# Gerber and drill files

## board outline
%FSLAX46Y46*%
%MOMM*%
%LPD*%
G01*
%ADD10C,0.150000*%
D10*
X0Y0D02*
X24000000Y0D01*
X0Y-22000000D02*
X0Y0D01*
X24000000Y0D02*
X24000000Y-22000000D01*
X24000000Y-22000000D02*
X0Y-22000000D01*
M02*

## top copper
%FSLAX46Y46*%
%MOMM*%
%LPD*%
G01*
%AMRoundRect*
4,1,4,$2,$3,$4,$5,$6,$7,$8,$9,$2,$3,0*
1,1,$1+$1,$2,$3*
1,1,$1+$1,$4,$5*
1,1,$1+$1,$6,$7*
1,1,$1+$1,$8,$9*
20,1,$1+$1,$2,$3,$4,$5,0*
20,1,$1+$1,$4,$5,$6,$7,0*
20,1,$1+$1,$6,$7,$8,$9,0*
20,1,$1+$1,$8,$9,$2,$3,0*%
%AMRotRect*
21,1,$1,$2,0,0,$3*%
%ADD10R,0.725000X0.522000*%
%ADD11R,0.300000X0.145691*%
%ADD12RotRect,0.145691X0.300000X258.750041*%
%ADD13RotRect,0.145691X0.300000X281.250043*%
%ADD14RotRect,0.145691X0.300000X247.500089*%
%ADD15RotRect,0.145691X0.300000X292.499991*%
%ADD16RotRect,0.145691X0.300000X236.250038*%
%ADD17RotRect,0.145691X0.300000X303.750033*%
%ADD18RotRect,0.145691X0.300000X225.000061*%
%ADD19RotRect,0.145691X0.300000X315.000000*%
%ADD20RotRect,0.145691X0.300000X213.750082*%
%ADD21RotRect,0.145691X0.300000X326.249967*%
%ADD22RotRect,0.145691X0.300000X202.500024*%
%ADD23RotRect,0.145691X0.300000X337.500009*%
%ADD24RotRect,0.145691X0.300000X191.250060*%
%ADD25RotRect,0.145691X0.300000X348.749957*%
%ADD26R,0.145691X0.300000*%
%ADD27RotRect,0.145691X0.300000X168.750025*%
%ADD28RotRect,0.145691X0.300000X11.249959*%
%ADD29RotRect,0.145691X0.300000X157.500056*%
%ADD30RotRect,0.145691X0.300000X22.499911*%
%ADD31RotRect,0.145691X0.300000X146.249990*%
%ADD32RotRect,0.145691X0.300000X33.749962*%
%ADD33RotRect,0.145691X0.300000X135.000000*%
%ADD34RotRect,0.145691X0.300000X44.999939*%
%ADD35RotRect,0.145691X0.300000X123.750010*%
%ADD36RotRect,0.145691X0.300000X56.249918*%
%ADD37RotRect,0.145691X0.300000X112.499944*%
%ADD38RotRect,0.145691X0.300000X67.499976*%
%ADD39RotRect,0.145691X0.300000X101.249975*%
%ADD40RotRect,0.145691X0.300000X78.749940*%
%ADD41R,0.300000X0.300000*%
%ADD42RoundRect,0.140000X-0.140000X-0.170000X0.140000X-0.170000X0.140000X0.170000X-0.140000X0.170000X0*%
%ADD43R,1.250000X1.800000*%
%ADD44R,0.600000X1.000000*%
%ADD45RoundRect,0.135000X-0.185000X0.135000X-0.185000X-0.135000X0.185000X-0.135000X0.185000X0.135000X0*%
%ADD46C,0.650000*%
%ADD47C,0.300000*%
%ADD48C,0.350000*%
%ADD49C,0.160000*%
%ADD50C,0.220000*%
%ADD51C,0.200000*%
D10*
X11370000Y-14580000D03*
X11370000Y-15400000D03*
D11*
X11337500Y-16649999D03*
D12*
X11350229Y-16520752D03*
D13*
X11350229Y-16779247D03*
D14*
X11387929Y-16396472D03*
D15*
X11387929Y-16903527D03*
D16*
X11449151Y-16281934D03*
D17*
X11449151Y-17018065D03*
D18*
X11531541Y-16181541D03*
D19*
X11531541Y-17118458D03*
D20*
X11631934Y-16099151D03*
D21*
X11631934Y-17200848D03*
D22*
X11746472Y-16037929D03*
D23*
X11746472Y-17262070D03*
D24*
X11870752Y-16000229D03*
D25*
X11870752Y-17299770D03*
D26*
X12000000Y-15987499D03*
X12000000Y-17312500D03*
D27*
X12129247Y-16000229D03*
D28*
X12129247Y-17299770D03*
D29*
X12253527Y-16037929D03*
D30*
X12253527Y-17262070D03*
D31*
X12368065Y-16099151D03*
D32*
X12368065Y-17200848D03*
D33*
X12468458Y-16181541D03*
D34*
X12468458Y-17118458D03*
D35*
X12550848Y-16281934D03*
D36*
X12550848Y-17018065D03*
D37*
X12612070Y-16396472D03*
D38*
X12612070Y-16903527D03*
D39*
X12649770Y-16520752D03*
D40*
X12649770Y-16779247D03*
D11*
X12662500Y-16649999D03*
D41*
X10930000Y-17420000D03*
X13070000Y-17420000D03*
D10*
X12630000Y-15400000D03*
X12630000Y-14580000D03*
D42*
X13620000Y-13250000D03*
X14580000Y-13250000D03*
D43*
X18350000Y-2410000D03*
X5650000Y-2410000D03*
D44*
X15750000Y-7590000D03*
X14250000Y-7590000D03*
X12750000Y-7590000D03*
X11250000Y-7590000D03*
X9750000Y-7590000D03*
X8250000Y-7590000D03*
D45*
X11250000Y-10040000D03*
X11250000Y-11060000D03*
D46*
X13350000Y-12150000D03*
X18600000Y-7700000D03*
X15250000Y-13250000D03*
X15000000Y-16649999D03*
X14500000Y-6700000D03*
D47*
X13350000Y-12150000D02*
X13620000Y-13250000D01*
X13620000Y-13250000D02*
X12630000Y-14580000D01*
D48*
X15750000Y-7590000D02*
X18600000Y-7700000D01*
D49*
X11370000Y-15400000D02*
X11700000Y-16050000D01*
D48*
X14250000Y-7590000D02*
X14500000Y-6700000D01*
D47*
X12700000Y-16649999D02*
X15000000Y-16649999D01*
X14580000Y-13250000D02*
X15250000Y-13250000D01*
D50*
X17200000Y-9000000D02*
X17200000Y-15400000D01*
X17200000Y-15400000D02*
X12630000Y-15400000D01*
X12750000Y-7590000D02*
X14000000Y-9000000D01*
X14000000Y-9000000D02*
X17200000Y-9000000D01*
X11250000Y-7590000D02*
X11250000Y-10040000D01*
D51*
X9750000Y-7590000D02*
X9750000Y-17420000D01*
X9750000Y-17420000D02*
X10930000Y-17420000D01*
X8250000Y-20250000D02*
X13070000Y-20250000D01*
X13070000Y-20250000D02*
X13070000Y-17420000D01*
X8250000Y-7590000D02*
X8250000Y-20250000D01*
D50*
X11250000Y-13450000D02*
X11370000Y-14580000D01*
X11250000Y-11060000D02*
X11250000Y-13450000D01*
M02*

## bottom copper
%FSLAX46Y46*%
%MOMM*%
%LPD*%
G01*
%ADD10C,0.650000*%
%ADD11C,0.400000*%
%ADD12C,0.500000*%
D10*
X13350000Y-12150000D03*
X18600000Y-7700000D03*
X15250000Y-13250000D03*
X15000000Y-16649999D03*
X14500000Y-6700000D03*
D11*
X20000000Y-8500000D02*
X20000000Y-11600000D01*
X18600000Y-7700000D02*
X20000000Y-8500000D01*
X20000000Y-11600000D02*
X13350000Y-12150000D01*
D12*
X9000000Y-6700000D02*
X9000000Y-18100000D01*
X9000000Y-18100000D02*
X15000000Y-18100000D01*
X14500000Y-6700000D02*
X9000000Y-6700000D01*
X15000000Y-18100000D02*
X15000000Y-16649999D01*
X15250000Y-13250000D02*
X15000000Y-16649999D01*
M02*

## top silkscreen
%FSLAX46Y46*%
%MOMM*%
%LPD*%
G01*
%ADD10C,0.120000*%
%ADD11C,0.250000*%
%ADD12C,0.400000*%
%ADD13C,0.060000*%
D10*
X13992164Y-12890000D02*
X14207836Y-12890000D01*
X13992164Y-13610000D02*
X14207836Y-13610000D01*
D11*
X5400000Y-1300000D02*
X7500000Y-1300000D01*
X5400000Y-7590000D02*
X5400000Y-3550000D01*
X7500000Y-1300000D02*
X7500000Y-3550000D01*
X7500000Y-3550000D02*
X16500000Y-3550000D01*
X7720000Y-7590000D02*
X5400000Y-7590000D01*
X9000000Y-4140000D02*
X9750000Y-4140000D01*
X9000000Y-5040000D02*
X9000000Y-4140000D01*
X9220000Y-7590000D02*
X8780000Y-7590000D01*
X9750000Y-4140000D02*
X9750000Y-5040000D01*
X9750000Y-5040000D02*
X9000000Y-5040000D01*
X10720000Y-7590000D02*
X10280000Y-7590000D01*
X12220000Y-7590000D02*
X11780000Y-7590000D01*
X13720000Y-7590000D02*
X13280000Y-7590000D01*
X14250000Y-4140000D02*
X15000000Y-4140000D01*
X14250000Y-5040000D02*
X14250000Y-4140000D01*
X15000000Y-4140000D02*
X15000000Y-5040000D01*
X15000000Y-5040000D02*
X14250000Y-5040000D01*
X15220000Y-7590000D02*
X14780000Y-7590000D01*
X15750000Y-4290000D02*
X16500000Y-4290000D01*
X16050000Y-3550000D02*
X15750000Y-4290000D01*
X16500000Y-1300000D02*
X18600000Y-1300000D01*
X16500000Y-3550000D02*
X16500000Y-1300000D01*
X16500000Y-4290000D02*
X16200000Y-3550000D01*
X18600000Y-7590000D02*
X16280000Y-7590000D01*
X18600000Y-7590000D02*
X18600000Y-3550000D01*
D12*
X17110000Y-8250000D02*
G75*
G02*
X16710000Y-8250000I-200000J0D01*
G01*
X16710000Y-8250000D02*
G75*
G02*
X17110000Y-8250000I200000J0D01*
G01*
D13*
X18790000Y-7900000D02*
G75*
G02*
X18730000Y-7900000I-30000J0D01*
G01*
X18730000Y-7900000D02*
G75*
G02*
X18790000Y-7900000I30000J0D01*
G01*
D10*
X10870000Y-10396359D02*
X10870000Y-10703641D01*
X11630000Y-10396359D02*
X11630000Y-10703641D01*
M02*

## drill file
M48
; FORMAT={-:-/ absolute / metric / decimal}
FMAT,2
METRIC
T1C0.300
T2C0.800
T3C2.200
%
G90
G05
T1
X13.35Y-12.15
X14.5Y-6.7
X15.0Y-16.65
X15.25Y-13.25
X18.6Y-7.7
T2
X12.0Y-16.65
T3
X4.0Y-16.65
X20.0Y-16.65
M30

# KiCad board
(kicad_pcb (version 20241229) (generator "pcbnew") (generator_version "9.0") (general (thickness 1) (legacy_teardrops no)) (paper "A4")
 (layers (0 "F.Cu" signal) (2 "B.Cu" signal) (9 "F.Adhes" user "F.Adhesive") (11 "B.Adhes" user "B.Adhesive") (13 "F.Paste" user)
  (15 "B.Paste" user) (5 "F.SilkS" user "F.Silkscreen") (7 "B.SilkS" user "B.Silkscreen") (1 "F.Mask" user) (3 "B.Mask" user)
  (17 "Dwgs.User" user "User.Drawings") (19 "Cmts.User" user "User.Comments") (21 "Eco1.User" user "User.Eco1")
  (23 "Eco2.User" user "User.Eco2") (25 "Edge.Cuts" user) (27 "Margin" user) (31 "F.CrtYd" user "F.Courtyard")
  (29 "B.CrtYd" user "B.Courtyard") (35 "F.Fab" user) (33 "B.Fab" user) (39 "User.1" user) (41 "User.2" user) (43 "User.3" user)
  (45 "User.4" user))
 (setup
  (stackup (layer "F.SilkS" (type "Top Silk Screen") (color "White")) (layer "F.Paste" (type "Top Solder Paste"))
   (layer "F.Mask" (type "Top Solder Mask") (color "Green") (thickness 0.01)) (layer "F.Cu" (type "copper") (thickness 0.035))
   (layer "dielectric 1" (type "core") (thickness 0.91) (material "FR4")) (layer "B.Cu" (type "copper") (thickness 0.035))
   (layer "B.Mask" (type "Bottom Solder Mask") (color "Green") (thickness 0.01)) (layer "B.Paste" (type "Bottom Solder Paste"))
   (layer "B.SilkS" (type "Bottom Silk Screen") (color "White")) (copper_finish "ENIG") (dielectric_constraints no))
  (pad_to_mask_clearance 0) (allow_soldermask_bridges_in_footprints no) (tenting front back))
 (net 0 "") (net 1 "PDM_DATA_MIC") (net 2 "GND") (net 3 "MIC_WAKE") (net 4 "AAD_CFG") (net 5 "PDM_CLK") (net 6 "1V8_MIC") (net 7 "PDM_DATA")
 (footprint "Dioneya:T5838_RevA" (layer "F.Cu") (at 12 16)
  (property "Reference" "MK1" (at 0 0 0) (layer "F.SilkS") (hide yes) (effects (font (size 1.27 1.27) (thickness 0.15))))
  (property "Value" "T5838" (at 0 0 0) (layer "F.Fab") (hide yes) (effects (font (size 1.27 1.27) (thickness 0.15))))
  (pad "" np_thru_hole circle (at 0 0.649999) (size 0.8 0.8) (drill 0.8) (layers "*.Cu" "*.Mask"))
  (pad "1" smd rect (at -0.63 -1.42 90) (size 0.522 0.725) (layers "F.Cu" "F.Mask" "F.Paste") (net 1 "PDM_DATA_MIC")
   (solder_paste_margin -0.05) (thermal_bridge_angle 45))
  (pad "2" smd rect (at -0.63 -0.6 90) (size 0.522 0.725) (layers "F.Cu" "F.Mask" "F.Paste") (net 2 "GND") (solder_paste_margin -0.05)
   (thermal_bridge_angle 45))
  (pad "3" smd rect (at -0.6625 0.649999 270) (size 0.145691 0.3) (layers "F.Cu" "F.Mask") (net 2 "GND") (thermal_bridge_angle 45))
  (pad "3" smd rect (at -0.649771 0.520752 258.750041) (size 0.145691 0.3) (layers "F.Cu" "F.Mask") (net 2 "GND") (thermal_bridge_angle 45))
  (pad "3" smd rect (at -0.649771 0.779247 281.250043) (size 0.145691 0.3) (layers "F.Cu" "F.Mask") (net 2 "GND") (thermal_bridge_angle 45))
  (pad "3" smd rect (at -0.612071 0.396472 247.500089) (size 0.145691 0.3) (layers "F.Cu" "F.Mask") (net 2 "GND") (thermal_bridge_angle 45))
  (pad "3" smd rect (at -0.612071 0.903527 292.499991) (size 0.145691 0.3) (layers "F.Cu" "F.Mask") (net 2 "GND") (thermal_bridge_angle 45))
  (pad "3" smd rect (at -0.550849 0.281934 236.250038) (size 0.145691 0.3) (layers "F.Cu" "F.Mask") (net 2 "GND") (thermal_bridge_angle 45))
  (pad "3" smd rect (at -0.550849 1.018065 303.750033) (size 0.145691 0.3) (layers "F.Cu" "F.Mask") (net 2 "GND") (thermal_bridge_angle 45))
  (pad "3" smd rect (at -0.468459 0.181541 225.000061) (size 0.145691 0.3) (layers "F.Cu" "F.Mask") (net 2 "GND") (thermal_bridge_angle 45))
  (pad "3" smd rect (at -0.468459 1.118458 315) (size 0.145691 0.3) (layers "F.Cu" "F.Mask") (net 2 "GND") (thermal_bridge_angle 45))
  (pad "3" smd rect (at -0.368066 0.099151 213.750082) (size 0.145691 0.3) (layers "F.Cu" "F.Mask") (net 2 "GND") (thermal_bridge_angle 45))
  (pad "3" smd rect (at -0.368066 1.200848 326.249967) (size 0.145691 0.3) (layers "F.Cu" "F.Mask") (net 2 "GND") (thermal_bridge_angle 45))
  (pad "3" smd rect (at -0.253528 0.037929 202.500024) (size 0.145691 0.3) (layers "F.Cu" "F.Mask") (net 2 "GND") (thermal_bridge_angle 45))
  (pad "3" smd rect (at -0.253528 1.26207 337.500009) (size 0.145691 0.3) (layers "F.Cu" "F.Mask") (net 2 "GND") (thermal_bridge_angle 45))
  (pad "3" smd rect (at -0.129248 0.000229 191.25006) (size 0.145691 0.3) (layers "F.Cu" "F.Mask") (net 2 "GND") (thermal_bridge_angle 45))
  (pad "3" smd rect (at -0.129248 1.29977 348.749957) (size 0.145691 0.3) (layers "F.Cu" "F.Mask") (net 2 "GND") (thermal_bridge_angle 45))
  (pad "3" smd rect (at 0 -0.012501 180) (size 0.145691 0.3) (layers "F.Cu" "F.Mask") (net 2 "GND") (thermal_bridge_angle 45))
  (pad "3" smd rect (at 0 1.3125) (size 0.145691 0.3) (layers "F.Cu" "F.Mask") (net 2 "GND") (thermal_bridge_angle 45))
  (pad "3" smd rect (at 0.129247 0.000229 168.750025) (size 0.145691 0.3) (layers "F.Cu" "F.Mask") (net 2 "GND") (thermal_bridge_angle 45))
  (pad "3" smd rect (at 0.129247 1.29977 11.249959) (size 0.145691 0.3) (layers "F.Cu" "F.Mask") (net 2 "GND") (thermal_bridge_angle 45))
  (pad "3" smd rect (at 0.253527 0.037929 157.500056) (size 0.145691 0.3) (layers "F.Cu" "F.Mask") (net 2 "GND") (thermal_bridge_angle 45))
  (pad "3" smd rect (at 0.253527 1.26207 22.499911) (size 0.145691 0.3) (layers "F.Cu" "F.Mask") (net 2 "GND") (thermal_bridge_angle 45))
  (pad "3" smd rect (at 0.368065 0.099151 146.24999) (size 0.145691 0.3) (layers "F.Cu" "F.Mask") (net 2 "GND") (thermal_bridge_angle 45))
  (pad "3" smd rect (at 0.368065 1.200848 33.749962) (size 0.145691 0.3) (layers "F.Cu" "F.Mask") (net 2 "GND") (thermal_bridge_angle 45))
  (pad "3" smd rect (at 0.468458 0.181541 135) (size 0.145691 0.3) (layers "F.Cu" "F.Mask") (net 2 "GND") (thermal_bridge_angle 45))
  (pad "3" smd rect (at 0.468458 1.118458 44.999939) (size 0.145691 0.3) (layers "F.Cu" "F.Mask") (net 2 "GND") (thermal_bridge_angle 45))
  (pad "3" smd rect (at 0.550848 0.281934 123.75001) (size 0.145691 0.3) (layers "F.Cu" "F.Mask") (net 2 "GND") (thermal_bridge_angle 45))
  (pad "3" smd rect (at 0.550848 1.018065 56.249918) (size 0.145691 0.3) (layers "F.Cu" "F.Mask") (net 2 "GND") (thermal_bridge_angle 45))
  (pad "3" smd rect (at 0.61207 0.396472 112.499944) (size 0.145691 0.3) (layers "F.Cu" "F.Mask") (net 2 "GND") (thermal_bridge_angle 45))
  (pad "3" smd rect (at 0.61207 0.903527 67.499976) (size 0.145691 0.3) (layers "F.Cu" "F.Mask") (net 2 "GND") (thermal_bridge_angle 45))
  (pad "3" smd rect (at 0.64977 0.520752 101.249975) (size 0.145691 0.3) (layers "F.Cu" "F.Mask") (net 2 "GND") (thermal_bridge_angle 45))
  (pad "3" smd rect (at 0.64977 0.779247 78.74994) (size 0.145691 0.3) (layers "F.Cu" "F.Mask") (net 2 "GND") (thermal_bridge_angle 45))
  (pad "3" smd rect (at 0.6625 0.649999 90) (size 0.145691 0.3) (layers "F.Cu" "F.Mask") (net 2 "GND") (thermal_bridge_angle 45))
  (pad "4" smd rect (at -1.07 1.42 90) (size 0.3 0.3) (layers "F.Cu" "F.Mask" "F.Paste") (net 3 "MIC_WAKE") (solder_paste_margin -0.015)
   (thermal_bridge_angle 45))
  (pad "5" smd rect (at 1.07 1.42 90) (size 0.3 0.3) (layers "F.Cu" "F.Mask" "F.Paste") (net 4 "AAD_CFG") (solder_paste_margin -0.015)
   (thermal_bridge_angle 45))
  (pad "6" smd rect (at 0.63 -0.6 90) (size 0.522 0.725) (layers "F.Cu" "F.Mask" "F.Paste") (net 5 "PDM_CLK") (solder_paste_margin -0.05)
   (thermal_bridge_angle 45))
  (pad "7" smd rect (at 0.63 -1.42 90) (size 0.522 0.725) (layers "F.Cu" "F.Mask" "F.Paste") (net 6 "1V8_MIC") (solder_paste_margin -0.05)
   (thermal_bridge_angle 45)))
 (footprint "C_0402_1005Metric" (layer "F.Cu") (at 14.1 13.25)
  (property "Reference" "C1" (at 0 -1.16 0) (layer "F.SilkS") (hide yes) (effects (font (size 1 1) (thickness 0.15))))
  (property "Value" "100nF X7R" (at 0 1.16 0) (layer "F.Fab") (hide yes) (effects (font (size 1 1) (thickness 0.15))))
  (fp_line (start -0.107836 -0.36) (end 0.107836 -0.36) (stroke (width 0.12) (type solid)) (layer "F.SilkS"))
  (fp_line (start -0.107836 0.36) (end 0.107836 0.36) (stroke (width 0.12) (type solid)) (layer "F.SilkS"))
  (pad "1" smd roundrect (at -0.48 0) (size 0.56 0.62) (layers "F.Cu" "F.Mask" "F.Paste") (roundrect_rratio 0.25) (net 6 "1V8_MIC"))
  (pad "2" smd roundrect (at 0.48 0) (size 0.56 0.62) (layers "F.Cu" "F.Mask" "F.Paste") (roundrect_rratio 0.25) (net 2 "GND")))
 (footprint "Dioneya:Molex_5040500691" (layer "F.Cu") (at 12 5 180)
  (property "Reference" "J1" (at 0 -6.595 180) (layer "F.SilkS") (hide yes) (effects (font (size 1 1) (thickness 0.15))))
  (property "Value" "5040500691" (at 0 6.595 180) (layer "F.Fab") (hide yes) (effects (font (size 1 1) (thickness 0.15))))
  (fp_line (start 6.6 3.7) (end 4.5 3.7) (stroke (width 0.25) (type solid)) (layer "F.SilkS"))
  (fp_line (start 6.6 -2.59) (end 6.6 1.45) (stroke (width 0.25) (type solid)) (layer "F.SilkS"))
  (fp_line (start 4.5 3.7) (end 4.5 1.45) (stroke (width 0.25) (type solid)) (layer "F.SilkS"))
  (fp_line (start 4.5 1.45) (end -4.5 1.45) (stroke (width 0.25) (type solid)) (layer "F.SilkS"))
  (fp_line (start 4.28 -2.59) (end 6.6 -2.59) (stroke (width 0.25) (type solid)) (layer "F.SilkS"))
  (fp_line (start 3 0.86) (end 2.25 0.86) (stroke (width 0.25) (type solid)) (layer "F.SilkS"))
  (fp_line (start 3 -0.04) (end 3 0.86) (stroke (width 0.25) (type solid)) (layer "F.SilkS"))
  (fp_line (start 2.78 -2.59) (end 3.22 -2.59) (stroke (width 0.25) (type solid)) (layer "F.SilkS"))
  (fp_line (start 2.25 0.86) (end 2.25 -0.04) (stroke (width 0.25) (type solid)) (layer "F.SilkS"))
  (fp_line (start 2.25 -0.04) (end 3 -0.04) (stroke (width 0.25) (type solid)) (layer "F.SilkS"))
  (fp_line (start 1.28 -2.59) (end 1.72 -2.59) (stroke (width 0.25) (type solid)) (layer "F.SilkS"))
  (fp_line (start -0.22 -2.59) (end 0.22 -2.59) (stroke (width 0.25) (type solid)) (layer "F.SilkS"))
  (fp_line (start -1.72 -2.59) (end -1.28 -2.59) (stroke (width 0.25) (type solid)) (layer "F.SilkS"))
  (fp_line (start -2.25 0.86) (end -3 0.86) (stroke (width 0.25) (type solid)) (layer "F.SilkS"))
  (fp_line (start -2.25 -0.04) (end -2.25 0.86) (stroke (width 0.25) (type solid)) (layer "F.SilkS"))
  (fp_line (start -3 0.86) (end -3 -0.04) (stroke (width 0.25) (type solid)) (layer "F.SilkS"))
  (fp_line (start -3 -0.04) (end -2.25 -0.04) (stroke (width 0.25) (type solid)) (layer "F.SilkS"))
  (fp_line (start -3.22 -2.59) (end -2.78 -2.59) (stroke (width 0.25) (type solid)) (layer "F.SilkS"))
  (fp_line (start -3.75 0.71) (end -4.5 0.71) (stroke (width 0.25) (type solid)) (layer "F.SilkS"))
  (fp_line (start -4.05 1.45) (end -3.75 0.71) (stroke (width 0.25) (type solid)) (layer "F.SilkS"))
  (fp_line (start -4.5 3.7) (end -6.6 3.7) (stroke (width 0.25) (type solid)) (layer "F.SilkS"))
  (fp_line (start -4.5 1.45) (end -4.5 3.7) (stroke (width 0.25) (type solid)) (layer "F.SilkS"))
  (fp_line (start -4.5 0.71) (end -4.2 1.45) (stroke (width 0.25) (type solid)) (layer "F.SilkS"))
  (fp_line (start -6.6 -2.59) (end -4.28 -2.59) (stroke (width 0.25) (type solid)) (layer "F.SilkS"))
  (fp_line (start -6.6 -2.59) (end -6.6 1.45) (stroke (width 0.25) (type solid)) (layer "F.SilkS"))
  (fp_circle (center -4.91 -3.25) (end -4.71 -3.25) (stroke (width 0.4) (type solid)) (fill no) (layer "F.SilkS"))
  (fp_circle (center -6.76 -2.9) (end -6.73 -2.9) (stroke (width 0.06) (type solid)) (fill no) (layer "F.SilkS"))
  (pad "" smd rect (at -6.35 2.59) (size 1.25 1.8) (layers "F.Cu" "F.Mask" "F.Paste"))
  (pad "" smd rect (at 6.35 2.59) (size 1.25 1.8) (layers "F.Cu" "F.Mask" "F.Paste"))
  (pad "1" smd rect (at -3.75 -2.59) (size 0.6 1) (layers "F.Cu" "F.Mask" "F.Paste") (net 6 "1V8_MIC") (solder_paste_margin 0))
  (pad "2" smd rect (at -2.25 -2.59) (size 0.6 1) (layers "F.Cu" "F.Mask" "F.Paste") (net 2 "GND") (solder_paste_margin 0))
  (pad "3" smd rect (at -0.75 -2.59) (size 0.6 1) (layers "F.Cu" "F.Mask" "F.Paste") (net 5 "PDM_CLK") (solder_paste_margin 0))
  (pad "4" smd rect (at 0.75 -2.59) (size 0.6 1) (layers "F.Cu" "F.Mask" "F.Paste") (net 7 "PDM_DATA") (solder_paste_margin 0))
  (pad "5" smd rect (at 2.25 -2.59) (size 0.6 1) (layers "F.Cu" "F.Mask" "F.Paste") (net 3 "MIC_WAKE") (solder_paste_margin 0))
  (pad "6" smd rect (at 3.75 -2.59) (size 0.6 1) (layers "F.Cu" "F.Mask" "F.Paste") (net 4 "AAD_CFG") (solder_paste_margin 0)))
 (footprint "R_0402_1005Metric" (layer "F.Cu") (at 11.25 10.55 -90)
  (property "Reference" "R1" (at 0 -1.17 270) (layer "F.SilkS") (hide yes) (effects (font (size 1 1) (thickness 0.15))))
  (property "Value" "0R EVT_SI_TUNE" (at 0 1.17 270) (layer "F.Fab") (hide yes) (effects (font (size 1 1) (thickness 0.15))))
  (fp_line (start -0.153641 0.38) (end 0.153641 0.38) (stroke (width 0.12) (type solid)) (layer "F.SilkS"))
  (fp_line (start -0.153641 -0.38) (end 0.153641 -0.38) (stroke (width 0.12) (type solid)) (layer "F.SilkS"))
  (pad "1" smd roundrect (at -0.51 0 270) (size 0.54 0.64) (layers "F.Cu" "F.Mask" "F.Paste") (roundrect_rratio 0.25) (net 7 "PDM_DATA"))
  (pad "2" smd roundrect (at 0.51 0 270) (size 0.54 0.64) (layers "F.Cu" "F.Mask" "F.Paste") (roundrect_rratio 0.25) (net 1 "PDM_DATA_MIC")))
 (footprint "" (layer "F.Cu") (at 4 16.649999)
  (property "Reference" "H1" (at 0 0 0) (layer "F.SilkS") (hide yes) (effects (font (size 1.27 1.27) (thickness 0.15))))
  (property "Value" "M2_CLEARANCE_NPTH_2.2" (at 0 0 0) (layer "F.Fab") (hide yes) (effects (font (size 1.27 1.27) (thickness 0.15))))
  (pad "" np_thru_hole circle (at 0 0) (size 2.2 2.2) (drill 2.2) (layers "*.Cu" "*.Mask")))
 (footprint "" (layer "F.Cu") (at 20 16.649999)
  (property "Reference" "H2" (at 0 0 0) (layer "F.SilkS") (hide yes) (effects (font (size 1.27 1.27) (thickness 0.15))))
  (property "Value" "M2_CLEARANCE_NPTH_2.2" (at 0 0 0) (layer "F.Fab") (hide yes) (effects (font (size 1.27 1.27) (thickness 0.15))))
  (pad "" np_thru_hole circle (at 0 0) (size 2.2 2.2) (drill 2.2) (layers "*.Cu" "*.Mask")))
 (gr_line (start 0 0) (end 24 0) (stroke (width 0.15) (type default)) (layer "Edge.Cuts"))
 (gr_line (start 0 22) (end 0 0) (stroke (width 0.15) (type default)) (layer "Edge.Cuts"))
 (gr_line (start 24 0) (end 24 22) (stroke (width 0.15) (type default)) (layer "Edge.Cuts"))
 (gr_line (start 24 22) (end 0 22) (stroke (width 0.15) (type default)) (layer "Edge.Cuts"))
 (segment (start 13.35 12.15) (end 13.62 13.25) (width 0.3) (layer "F.Cu") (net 6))
 (segment (start 13.62 13.25) (end 12.63 14.58) (width 0.3) (layer "F.Cu") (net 6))
 (segment (start 15.75 7.59) (end 18.6 7.7) (width 0.35) (layer "F.Cu") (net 6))
 (via (at 13.35 12.15) (size 0.65) (drill 0.3) (layers "F.Cu" "B.Cu") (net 6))
 (via (at 18.6 7.7) (size 0.65) (drill 0.3) (layers "F.Cu" "B.Cu") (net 6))
 (segment (start 20 8.5) (end 20 11.6) (width 0.4) (layer "B.Cu") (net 6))
 (segment (start 18.6 7.7) (end 20 8.5) (width 0.4) (layer "B.Cu") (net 6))
 (segment (start 20 11.6) (end 13.35 12.15) (width 0.4) (layer "B.Cu") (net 6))
 (segment (start 11.37 15.4) (end 11.7 16.05) (width 0.16) (layer "F.Cu") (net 2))
 (segment (start 14.25 7.59) (end 14.5 6.7) (width 0.35) (layer "F.Cu") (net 2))
 (segment (start 12.7 16.649999) (end 15 16.649999) (width 0.3) (layer "F.Cu") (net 2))
 (segment (start 14.58 13.25) (end 15.25 13.25) (width 0.3) (layer "F.Cu") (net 2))
 (via (at 15.25 13.25) (size 0.65) (drill 0.3) (layers "F.Cu" "B.Cu") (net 2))
 (via (at 15 16.649999) (size 0.65) (drill 0.3) (layers "F.Cu" "B.Cu") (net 2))
 (via (at 14.5 6.7) (size 0.65) (drill 0.3) (layers "F.Cu" "B.Cu") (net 2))
 (segment (start 9 6.7) (end 9 18.1) (width 0.5) (layer "B.Cu") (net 2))
 (segment (start 9 18.1) (end 15 18.1) (width 0.5) (layer "B.Cu") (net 2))
 (segment (start 14.5 6.7) (end 9 6.7) (width 0.5) (layer "B.Cu") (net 2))
 (segment (start 15 18.1) (end 15 16.649999) (width 0.5) (layer "B.Cu") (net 2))
 (segment (start 15.25 13.25) (end 15 16.649999) (width 0.5) (layer "B.Cu") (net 2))
 (segment (start 17.2 9) (end 17.2 15.4) (width 0.22) (layer "F.Cu") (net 5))
 (segment (start 17.2 15.4) (end 12.63 15.4) (width 0.22) (layer "F.Cu") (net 5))
 (segment (start 12.75 7.59) (end 14 9) (width 0.22) (layer "F.Cu") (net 5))
 (segment (start 14 9) (end 17.2 9) (width 0.22) (layer "F.Cu") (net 5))
 (segment (start 11.25 7.59) (end 11.25 10.04) (width 0.22) (layer "F.Cu") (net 7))
 (segment (start 9.75 7.59) (end 9.75 17.42) (width 0.2) (layer "F.Cu") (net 3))
 (segment (start 9.75 17.42) (end 10.93 17.42) (width 0.2) (layer "F.Cu") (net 3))
 (segment (start 8.25 20.25) (end 13.07 20.25) (width 0.2) (layer "F.Cu") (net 4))
 (segment (start 13.07 20.25) (end 13.07 17.42) (width 0.2) (layer "F.Cu") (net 4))
 (segment (start 8.25 7.59) (end 8.25 20.25) (width 0.2) (layer "F.Cu") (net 4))
 (segment (start 11.25 13.45) (end 11.37 14.58) (width 0.22) (layer "F.Cu") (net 1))
 (segment (start 11.25 11.06) (end 11.25 13.45) (width 0.22) (layer "F.Cu") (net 1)))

